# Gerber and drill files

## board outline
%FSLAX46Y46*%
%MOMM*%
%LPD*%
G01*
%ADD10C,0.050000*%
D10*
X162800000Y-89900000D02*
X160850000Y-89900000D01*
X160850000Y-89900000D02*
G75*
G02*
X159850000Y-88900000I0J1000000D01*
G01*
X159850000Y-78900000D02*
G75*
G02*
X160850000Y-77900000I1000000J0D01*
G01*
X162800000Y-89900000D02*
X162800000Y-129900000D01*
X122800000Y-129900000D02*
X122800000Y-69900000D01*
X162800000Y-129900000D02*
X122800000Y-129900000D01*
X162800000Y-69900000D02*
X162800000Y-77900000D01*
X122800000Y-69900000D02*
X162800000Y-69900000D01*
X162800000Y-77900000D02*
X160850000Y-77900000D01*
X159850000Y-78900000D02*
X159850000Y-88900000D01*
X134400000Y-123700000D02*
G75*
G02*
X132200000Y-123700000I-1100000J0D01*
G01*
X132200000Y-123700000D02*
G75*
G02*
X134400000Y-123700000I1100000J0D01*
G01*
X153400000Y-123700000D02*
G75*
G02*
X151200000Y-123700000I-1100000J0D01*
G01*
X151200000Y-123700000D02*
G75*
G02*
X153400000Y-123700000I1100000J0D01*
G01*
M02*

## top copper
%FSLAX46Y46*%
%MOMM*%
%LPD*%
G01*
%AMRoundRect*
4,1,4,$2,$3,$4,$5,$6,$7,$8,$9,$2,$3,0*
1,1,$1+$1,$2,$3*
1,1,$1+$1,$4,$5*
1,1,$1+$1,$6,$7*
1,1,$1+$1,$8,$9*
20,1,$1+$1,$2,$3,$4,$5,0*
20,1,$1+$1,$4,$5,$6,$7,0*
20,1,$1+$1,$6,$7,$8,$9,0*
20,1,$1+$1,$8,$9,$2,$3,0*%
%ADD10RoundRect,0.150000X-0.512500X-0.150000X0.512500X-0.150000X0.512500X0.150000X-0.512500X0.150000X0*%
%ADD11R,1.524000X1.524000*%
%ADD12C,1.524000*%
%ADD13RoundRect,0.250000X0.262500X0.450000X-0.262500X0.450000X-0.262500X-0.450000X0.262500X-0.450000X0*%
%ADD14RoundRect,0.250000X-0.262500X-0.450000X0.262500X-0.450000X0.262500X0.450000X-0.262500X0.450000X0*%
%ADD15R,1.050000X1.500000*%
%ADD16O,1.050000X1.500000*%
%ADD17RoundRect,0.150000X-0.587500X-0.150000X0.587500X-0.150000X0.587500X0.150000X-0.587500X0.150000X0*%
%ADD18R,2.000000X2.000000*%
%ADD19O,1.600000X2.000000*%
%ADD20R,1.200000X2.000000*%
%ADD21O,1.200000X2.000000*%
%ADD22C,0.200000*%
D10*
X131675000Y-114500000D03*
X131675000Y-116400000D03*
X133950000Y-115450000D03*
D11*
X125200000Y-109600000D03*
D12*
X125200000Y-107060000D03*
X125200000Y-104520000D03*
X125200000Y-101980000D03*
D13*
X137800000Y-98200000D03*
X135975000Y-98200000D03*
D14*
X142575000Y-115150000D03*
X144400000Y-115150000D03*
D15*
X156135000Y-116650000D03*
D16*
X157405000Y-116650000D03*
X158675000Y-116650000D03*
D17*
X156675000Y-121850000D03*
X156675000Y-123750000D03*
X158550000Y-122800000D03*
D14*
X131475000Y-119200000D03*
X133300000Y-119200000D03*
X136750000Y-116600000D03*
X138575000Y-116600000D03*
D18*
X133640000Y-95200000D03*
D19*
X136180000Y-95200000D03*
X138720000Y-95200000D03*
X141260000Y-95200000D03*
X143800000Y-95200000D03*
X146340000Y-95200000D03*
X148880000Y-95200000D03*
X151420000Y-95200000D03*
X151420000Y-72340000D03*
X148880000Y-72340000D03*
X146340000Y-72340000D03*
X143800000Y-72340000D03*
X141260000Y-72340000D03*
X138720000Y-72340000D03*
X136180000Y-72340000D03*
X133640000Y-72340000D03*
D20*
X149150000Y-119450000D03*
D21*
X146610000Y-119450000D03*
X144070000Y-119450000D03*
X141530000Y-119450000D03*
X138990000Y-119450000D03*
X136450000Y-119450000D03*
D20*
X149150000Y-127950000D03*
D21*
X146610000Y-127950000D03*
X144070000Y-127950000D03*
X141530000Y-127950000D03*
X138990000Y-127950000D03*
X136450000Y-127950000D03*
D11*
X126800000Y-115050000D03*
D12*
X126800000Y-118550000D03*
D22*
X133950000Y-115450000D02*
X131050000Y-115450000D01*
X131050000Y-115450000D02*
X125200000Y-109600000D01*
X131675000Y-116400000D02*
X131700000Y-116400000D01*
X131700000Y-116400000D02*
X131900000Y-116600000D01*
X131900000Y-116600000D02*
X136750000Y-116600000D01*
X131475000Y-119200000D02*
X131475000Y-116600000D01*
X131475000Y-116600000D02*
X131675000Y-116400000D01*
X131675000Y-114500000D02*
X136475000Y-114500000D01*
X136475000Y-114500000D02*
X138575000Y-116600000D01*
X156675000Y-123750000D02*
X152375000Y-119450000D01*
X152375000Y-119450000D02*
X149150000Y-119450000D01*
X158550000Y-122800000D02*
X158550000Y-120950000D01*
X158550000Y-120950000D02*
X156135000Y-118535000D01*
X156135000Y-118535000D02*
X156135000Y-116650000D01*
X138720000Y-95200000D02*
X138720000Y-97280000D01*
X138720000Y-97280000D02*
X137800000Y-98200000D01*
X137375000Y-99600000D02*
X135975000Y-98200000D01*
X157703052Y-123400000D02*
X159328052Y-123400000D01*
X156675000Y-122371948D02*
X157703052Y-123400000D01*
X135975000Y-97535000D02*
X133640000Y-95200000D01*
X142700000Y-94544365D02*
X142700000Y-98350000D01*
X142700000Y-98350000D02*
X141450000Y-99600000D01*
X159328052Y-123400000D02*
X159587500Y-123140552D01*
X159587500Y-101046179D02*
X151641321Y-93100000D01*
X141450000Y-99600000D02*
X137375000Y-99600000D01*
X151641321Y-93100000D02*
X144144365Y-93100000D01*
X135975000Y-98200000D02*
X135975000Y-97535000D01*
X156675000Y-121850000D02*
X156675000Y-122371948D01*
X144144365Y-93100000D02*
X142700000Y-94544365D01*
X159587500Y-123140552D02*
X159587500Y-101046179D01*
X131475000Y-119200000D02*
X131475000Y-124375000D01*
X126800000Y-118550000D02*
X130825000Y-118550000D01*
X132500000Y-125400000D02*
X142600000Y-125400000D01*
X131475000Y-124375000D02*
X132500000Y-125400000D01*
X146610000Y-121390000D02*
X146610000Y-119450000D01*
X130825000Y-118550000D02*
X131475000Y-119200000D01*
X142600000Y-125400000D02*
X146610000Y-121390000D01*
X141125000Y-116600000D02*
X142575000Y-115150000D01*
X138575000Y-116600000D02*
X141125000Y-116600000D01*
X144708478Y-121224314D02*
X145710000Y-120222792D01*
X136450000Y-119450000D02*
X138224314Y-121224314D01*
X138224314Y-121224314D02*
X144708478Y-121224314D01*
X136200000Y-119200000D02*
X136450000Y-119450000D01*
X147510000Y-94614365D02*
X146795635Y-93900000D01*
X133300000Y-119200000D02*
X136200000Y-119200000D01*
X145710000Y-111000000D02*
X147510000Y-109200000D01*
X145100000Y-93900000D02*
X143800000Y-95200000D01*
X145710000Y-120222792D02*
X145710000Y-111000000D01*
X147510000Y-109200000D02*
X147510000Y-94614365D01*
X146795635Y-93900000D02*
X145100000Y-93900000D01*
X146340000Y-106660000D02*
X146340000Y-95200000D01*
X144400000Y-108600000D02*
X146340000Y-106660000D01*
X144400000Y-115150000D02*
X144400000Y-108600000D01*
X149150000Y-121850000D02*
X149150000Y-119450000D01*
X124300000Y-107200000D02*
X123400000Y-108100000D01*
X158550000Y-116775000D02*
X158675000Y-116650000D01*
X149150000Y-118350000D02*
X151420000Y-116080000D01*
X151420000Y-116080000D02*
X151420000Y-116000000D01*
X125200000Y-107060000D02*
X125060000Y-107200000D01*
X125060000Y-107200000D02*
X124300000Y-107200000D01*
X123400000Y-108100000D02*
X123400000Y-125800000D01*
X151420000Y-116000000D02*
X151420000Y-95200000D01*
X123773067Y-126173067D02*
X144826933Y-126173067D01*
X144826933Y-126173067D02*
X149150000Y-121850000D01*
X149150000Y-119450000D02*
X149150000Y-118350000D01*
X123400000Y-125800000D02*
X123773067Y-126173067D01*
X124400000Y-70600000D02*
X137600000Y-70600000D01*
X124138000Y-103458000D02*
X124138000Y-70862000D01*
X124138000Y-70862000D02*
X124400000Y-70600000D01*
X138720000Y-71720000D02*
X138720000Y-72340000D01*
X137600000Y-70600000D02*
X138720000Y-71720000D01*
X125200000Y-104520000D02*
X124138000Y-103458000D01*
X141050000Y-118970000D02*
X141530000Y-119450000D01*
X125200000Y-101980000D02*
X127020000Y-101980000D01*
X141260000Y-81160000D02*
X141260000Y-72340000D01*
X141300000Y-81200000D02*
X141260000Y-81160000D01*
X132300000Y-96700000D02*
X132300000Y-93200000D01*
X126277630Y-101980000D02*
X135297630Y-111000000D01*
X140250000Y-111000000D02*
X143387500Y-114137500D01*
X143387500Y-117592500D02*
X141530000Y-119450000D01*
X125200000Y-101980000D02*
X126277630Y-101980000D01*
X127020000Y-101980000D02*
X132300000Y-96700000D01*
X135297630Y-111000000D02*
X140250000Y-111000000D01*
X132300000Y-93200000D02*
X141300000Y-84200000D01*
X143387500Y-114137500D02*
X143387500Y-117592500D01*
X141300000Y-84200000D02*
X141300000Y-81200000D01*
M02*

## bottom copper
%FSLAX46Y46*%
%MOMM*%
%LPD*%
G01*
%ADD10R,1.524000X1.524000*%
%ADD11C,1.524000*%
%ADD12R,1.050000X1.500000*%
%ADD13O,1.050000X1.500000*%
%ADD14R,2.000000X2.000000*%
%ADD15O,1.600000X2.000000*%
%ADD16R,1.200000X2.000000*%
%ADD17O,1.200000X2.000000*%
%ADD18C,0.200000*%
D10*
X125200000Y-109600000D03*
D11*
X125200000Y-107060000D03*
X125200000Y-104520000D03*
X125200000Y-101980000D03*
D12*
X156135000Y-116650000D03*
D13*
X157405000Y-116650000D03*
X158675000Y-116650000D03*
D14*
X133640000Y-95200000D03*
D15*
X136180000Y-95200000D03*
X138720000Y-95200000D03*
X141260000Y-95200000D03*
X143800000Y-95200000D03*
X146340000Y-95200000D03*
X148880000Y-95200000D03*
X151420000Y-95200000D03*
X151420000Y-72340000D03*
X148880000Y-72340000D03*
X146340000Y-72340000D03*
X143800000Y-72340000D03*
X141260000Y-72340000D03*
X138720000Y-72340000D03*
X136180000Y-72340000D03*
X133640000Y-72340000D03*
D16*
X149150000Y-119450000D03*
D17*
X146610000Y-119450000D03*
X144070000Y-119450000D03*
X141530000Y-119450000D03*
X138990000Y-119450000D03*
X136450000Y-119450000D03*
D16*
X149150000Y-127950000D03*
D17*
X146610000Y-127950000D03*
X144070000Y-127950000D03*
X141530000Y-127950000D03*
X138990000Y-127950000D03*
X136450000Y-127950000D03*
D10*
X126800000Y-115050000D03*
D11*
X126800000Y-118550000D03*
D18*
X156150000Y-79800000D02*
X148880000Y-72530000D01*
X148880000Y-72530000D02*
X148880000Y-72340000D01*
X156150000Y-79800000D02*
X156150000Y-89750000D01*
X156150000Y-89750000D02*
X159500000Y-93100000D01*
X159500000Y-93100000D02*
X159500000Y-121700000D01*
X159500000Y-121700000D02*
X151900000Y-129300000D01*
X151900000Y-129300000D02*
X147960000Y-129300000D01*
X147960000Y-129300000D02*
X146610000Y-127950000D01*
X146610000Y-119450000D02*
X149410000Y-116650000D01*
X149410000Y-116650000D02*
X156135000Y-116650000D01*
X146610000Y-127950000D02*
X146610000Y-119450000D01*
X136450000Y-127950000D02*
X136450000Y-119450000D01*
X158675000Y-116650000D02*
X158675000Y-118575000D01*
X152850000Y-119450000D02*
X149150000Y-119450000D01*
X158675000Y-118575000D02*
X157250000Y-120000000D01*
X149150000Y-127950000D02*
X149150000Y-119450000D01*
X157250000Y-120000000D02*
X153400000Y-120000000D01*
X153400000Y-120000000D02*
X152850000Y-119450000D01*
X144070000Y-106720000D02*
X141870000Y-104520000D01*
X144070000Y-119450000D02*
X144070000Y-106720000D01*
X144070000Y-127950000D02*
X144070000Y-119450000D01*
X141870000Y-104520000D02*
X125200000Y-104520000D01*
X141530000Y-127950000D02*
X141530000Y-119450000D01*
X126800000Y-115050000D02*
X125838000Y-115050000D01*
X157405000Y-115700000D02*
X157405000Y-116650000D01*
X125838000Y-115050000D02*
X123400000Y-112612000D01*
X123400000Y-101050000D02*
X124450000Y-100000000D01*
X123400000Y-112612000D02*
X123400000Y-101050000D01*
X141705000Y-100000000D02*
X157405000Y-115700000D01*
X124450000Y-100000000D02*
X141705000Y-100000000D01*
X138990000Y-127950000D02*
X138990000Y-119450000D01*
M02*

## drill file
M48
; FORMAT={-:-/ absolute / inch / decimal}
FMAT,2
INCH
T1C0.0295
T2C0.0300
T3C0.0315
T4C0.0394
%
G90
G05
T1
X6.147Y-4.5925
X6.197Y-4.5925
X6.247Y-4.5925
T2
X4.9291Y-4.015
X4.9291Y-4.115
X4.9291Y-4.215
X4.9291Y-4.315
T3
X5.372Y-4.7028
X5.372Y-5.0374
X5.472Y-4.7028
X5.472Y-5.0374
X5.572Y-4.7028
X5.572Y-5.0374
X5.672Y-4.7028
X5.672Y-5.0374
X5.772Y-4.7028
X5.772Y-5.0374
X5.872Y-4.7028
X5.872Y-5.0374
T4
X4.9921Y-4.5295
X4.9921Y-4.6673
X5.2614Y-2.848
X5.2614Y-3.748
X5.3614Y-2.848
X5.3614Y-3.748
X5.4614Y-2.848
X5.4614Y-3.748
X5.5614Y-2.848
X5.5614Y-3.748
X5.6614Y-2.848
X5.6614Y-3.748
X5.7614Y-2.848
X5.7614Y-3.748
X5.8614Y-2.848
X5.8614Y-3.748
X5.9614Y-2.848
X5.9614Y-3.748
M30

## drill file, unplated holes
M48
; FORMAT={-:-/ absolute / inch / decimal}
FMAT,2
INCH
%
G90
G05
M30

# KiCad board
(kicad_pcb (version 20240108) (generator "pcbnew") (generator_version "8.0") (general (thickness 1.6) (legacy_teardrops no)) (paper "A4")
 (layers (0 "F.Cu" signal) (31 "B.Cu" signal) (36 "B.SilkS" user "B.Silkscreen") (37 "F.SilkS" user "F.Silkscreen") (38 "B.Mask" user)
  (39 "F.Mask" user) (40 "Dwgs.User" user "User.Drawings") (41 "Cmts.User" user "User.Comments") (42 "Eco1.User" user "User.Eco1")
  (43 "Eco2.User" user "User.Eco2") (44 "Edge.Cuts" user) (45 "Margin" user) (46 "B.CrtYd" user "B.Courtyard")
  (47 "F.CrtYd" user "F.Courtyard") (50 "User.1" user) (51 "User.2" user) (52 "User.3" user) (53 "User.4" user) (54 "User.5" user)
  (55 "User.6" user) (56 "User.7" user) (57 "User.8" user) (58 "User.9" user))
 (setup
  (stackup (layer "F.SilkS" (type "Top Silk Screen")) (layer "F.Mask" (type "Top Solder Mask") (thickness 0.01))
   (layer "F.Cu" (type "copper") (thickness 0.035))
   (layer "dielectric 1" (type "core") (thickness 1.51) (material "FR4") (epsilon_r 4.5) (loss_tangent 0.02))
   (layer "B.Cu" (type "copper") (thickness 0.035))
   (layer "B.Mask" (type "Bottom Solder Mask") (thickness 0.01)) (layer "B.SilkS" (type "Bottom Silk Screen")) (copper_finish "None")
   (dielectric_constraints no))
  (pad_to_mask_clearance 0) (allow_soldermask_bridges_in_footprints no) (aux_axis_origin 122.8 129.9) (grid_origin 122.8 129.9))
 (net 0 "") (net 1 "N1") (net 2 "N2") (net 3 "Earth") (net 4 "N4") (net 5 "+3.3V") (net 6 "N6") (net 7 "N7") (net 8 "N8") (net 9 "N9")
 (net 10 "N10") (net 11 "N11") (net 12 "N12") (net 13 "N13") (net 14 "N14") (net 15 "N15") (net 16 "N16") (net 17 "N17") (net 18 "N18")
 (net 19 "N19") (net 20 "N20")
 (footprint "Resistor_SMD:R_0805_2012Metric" (layer "F.Cu") (at 143.4875 115.15)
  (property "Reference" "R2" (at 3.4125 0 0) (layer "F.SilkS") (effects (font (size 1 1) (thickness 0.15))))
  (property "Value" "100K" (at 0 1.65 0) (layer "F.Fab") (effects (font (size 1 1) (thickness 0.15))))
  (pad "1" smd roundrect (at -0.9125 0) (size 1.025 1.4) (layers "F.Cu" "F.Paste" "F.Mask") (roundrect_rratio 0.243902) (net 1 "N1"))
  (pad "2" smd roundrect (at 0.9125 0) (size 1.025 1.4) (layers "F.Cu" "F.Paste" "F.Mask") (roundrect_rratio 0.243902) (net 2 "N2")))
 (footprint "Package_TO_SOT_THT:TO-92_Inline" (layer "F.Cu") (at 156.135 116.65)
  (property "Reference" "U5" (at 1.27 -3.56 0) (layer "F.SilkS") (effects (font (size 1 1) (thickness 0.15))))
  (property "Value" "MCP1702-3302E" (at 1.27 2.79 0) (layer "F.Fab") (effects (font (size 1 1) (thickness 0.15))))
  (pad "1" thru_hole rect (at 0 0) (size 1.05 1.5) (drill 0.75) (layers "*.Cu" "*.Mask") (remove_unused_layers no) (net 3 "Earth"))
  (pad "2" thru_hole oval (at 1.27 0) (size 1.05 1.5) (drill 0.75) (layers "*.Cu" "*.Mask") (remove_unused_layers no) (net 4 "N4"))
  (pad "3" thru_hole oval (at 2.54 0) (size 1.05 1.5) (drill 0.75) (layers "*.Cu" "*.Mask") (remove_unused_layers no) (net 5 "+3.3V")))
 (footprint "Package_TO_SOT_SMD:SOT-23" (layer "F.Cu") (at 157.6125 122.8)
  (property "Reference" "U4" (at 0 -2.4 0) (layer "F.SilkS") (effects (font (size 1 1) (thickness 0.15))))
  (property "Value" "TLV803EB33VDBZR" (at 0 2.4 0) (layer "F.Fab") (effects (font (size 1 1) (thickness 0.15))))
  (pad "1" smd roundrect (at -0.9375 -0.95) (size 1.475 0.6) (layers "F.Cu" "F.Paste" "F.Mask") (roundrect_rratio 0.25) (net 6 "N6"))
  (pad "2" smd roundrect (at -0.9375 0.95) (size 1.475 0.6) (layers "F.Cu" "F.Paste" "F.Mask") (roundrect_rratio 0.25) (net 5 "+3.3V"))
  (pad "3" smd roundrect (at 0.9375 0) (size 1.475 0.6) (layers "F.Cu" "F.Paste" "F.Mask") (roundrect_rratio 0.25) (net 3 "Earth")))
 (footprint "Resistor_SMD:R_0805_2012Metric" (layer "F.Cu") (at 132.3875 119.2)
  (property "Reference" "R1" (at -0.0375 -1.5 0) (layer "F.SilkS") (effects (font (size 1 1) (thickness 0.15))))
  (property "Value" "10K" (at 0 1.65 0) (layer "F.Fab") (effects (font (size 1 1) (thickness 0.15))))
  (pad "1" smd roundrect (at -0.9125 0) (size 1.025 1.4) (layers "F.Cu" "F.Paste" "F.Mask") (roundrect_rratio 0.243902) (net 3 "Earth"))
  (pad "2" smd roundrect (at 0.9125 0) (size 1.025 1.4) (layers "F.Cu" "F.Paste" "F.Mask") (roundrect_rratio 0.243902) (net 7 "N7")))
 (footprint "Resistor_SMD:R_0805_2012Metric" (layer "F.Cu") (at 137.6625 116.6)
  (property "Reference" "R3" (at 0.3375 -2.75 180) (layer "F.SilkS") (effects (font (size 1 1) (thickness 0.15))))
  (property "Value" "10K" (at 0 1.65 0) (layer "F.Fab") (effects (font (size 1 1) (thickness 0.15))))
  (pad "1" smd roundrect (at -0.9125 0) (size 1.025 1.4) (layers "F.Cu" "F.Paste" "F.Mask") (roundrect_rratio 0.243902) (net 3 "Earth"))
  (pad "2" smd roundrect (at 0.9125 0) (size 1.025 1.4) (layers "F.Cu" "F.Paste" "F.Mask") (roundrect_rratio 0.243902) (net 1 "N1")))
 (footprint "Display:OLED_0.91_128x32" (layer "F.Cu") (at 125.1732 109.5902)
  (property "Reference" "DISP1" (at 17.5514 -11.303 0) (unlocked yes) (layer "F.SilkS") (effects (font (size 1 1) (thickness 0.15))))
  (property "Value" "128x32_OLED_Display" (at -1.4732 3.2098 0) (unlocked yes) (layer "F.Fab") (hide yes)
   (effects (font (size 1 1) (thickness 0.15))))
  (pad "1" thru_hole rect (at 0.0268 0.0098) (size 1.524 1.524) (drill 0.762) (layers "*.Cu" "*.Mask") (remove_unused_layers no)
   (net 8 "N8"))
  (pad "2" thru_hole circle (at 0.0268 -2.5302) (size 1.524 1.524) (drill 0.762) (layers "*.Cu" "*.Mask") (remove_unused_layers no)
   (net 5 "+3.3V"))
  (pad "3" thru_hole circle (at 0.0268 -5.0702) (size 1.524 1.524) (drill 0.762) (layers "*.Cu" "*.Mask") (remove_unused_layers no)
   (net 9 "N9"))
  (pad "4" thru_hole circle (at 0.0268 -7.6102) (size 1.524 1.524) (drill 0.762) (layers "*.Cu" "*.Mask") (remove_unused_layers no)
   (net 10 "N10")))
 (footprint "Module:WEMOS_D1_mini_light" (layer "F.Cu") (at 133.64 95.2 90)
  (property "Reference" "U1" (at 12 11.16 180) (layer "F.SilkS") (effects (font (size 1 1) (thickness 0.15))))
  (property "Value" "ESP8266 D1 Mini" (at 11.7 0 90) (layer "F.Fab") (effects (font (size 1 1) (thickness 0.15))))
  (pad "1" thru_hole rect (at 0 0 90) (size 2 2) (drill 1) (layers "*.Cu" "*.Mask") (remove_unused_layers no) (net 6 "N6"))
  (pad "2" thru_hole oval (at 0 2.54 90) (size 2 1.6) (drill 1) (layers "*.Cu" "*.Mask") (remove_unused_layers no) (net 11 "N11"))
  (pad "3" thru_hole oval (at 0 5.08 90) (size 2 1.6) (drill 1) (layers "*.Cu" "*.Mask") (remove_unused_layers no) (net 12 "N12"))
  (pad "4" thru_hole oval (at 0 7.62 90) (size 2 1.6) (drill 1) (layers "*.Cu" "*.Mask") (remove_unused_layers no) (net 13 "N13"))
  (pad "5" thru_hole oval (at 0 10.16 90) (size 2 1.6) (drill 1) (layers "*.Cu" "*.Mask") (remove_unused_layers no) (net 7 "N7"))
  (pad "6" thru_hole oval (at 0 12.7 90) (size 2 1.6) (drill 1) (layers "*.Cu" "*.Mask") (remove_unused_layers no) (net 2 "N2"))
  (pad "7" thru_hole oval (at 0 15.24 90) (size 2 1.6) (drill 1) (layers "*.Cu" "*.Mask") (remove_unused_layers no) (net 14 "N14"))
  (pad "8" thru_hole oval (at 0 17.78 90) (size 2 1.6) (drill 1) (layers "*.Cu" "*.Mask") (remove_unused_layers no) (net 5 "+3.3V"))
  (pad "9" thru_hole oval (at 22.86 17.78 90) (size 2 1.6) (drill 1) (layers "*.Cu" "*.Mask") (remove_unused_layers no) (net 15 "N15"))
  (pad "10" thru_hole oval (at 22.86 15.24 90) (size 2 1.6) (drill 1) (layers "*.Cu" "*.Mask") (remove_unused_layers no) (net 3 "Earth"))
  (pad "11" thru_hole oval (at 22.86 12.7 90) (size 2 1.6) (drill 1) (layers "*.Cu" "*.Mask") (remove_unused_layers no) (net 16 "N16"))
  (pad "12" thru_hole oval (at 22.86 10.16 90) (size 2 1.6) (drill 1) (layers "*.Cu" "*.Mask") (remove_unused_layers no) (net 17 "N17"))
  (pad "13" thru_hole oval (at 22.86 7.62 90) (size 2 1.6) (drill 1) (layers "*.Cu" "*.Mask") (remove_unused_layers no) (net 10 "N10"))
  (pad "14" thru_hole oval (at 22.86 5.08 90) (size 2 1.6) (drill 1) (layers "*.Cu" "*.Mask") (remove_unused_layers no) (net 9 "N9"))
  (pad "15" thru_hole oval (at 22.86 2.54 90) (size 2 1.6) (drill 1) (layers "*.Cu" "*.Mask") (remove_unused_layers no) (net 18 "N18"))
  (pad "16" thru_hole oval (at 22.86 0 90) (size 2 1.6) (drill 1) (layers "*.Cu" "*.Mask") (remove_unused_layers no) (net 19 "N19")))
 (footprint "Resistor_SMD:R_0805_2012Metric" (layer "F.Cu") (at 136.8875 98.2 180)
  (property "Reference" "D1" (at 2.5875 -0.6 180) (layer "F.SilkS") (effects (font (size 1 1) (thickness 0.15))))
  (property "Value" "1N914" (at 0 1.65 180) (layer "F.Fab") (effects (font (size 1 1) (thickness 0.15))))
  (pad "1" smd roundrect (at -0.9125 0 180) (size 1.025 1.4) (layers "F.Cu" "F.Paste" "F.Mask") (roundrect_rratio 0.243902) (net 12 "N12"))
  (pad "2" smd roundrect (at 0.9125 0 180) (size 1.025 1.4) (layers "F.Cu" "F.Paste" "F.Mask") (roundrect_rratio 0.243902) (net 6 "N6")))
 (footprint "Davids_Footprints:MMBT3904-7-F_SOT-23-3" (layer "F.Cu") (at 132.8125 115.45)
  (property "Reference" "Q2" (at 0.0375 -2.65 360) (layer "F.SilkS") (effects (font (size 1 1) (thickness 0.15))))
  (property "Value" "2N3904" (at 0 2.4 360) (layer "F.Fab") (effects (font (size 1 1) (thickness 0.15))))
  (pad "1" smd roundrect (at -1.1375 -0.95) (size 1.325 0.6) (layers "F.Cu" "F.Paste" "F.Mask") (roundrect_rratio 0.25) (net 1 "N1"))
  (pad "2" smd roundrect (at -1.1375 0.95) (size 1.325 0.6) (layers "F.Cu" "F.Paste" "F.Mask") (roundrect_rratio 0.25) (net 3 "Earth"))
  (pad "3" smd roundrect (at 1.1375 0) (size 1.325 0.6) (layers "F.Cu" "F.Paste" "F.Mask") (roundrect_rratio 0.25) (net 8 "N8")))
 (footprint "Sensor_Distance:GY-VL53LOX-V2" (layer "F.Cu") (at 142.8 119.45 180)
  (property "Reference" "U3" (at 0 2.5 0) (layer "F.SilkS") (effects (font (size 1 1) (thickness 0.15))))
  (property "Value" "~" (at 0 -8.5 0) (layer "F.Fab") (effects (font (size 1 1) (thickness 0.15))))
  (pad "1" thru_hole rect (at -6.35 0 180) (size 1.2 2) (drill 0.8) (layers "*.Cu" "*.Mask") (remove_unused_layers no) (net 5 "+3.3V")
   (thermal_bridge_angle 45))
  (pad "2" thru_hole oval (at -3.81 0 180) (size 1.2 2) (drill 0.8) (layers "*.Cu" "*.Mask") (remove_unused_layers no) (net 3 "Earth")
   (thermal_bridge_angle 45))
  (pad "3" thru_hole oval (at -1.27 0 180) (size 1.2 2) (drill 0.8) (layers "*.Cu" "*.Mask") (remove_unused_layers no) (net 9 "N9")
   (thermal_bridge_angle 45))
  (pad "4" thru_hole oval (at 1.27 0 180) (size 1.2 2) (drill 0.8) (layers "*.Cu" "*.Mask") (remove_unused_layers no) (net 10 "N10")
   (thermal_bridge_angle 45))
  (pad "5" thru_hole oval (at 3.81 0 180) (size 1.2 2) (drill 0.8) (layers "*.Cu" "*.Mask") (remove_unused_layers no) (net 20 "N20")
   (thermal_bridge_angle 45))
  (pad "6" thru_hole oval (at 6.35 0 180) (size 1.2 2) (drill 0.8) (layers "*.Cu" "*.Mask") (remove_unused_layers no) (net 7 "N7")
   (thermal_bridge_angle 45)))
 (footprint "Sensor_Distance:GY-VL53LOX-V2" (layer "B.Cu") (at 142.8 127.95 180)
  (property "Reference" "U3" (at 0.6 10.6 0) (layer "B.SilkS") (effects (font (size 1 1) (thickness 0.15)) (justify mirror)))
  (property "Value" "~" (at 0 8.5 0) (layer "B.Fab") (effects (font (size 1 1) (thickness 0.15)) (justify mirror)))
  (pad "1" thru_hole rect (at -6.35 0 180) (size 1.2 2) (drill 0.8) (layers "*.Cu" "*.Mask") (remove_unused_layers no) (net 5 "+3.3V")
   (thermal_bridge_angle 45))
  (pad "2" thru_hole oval (at -3.81 0 180) (size 1.2 2) (drill 0.8) (layers "*.Cu" "*.Mask") (remove_unused_layers no) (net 3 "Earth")
   (thermal_bridge_angle 45))
  (pad "3" thru_hole oval (at -1.27 0 180) (size 1.2 2) (drill 0.8) (layers "*.Cu" "*.Mask") (remove_unused_layers no) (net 9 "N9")
   (thermal_bridge_angle 45))
  (pad "4" thru_hole oval (at 1.27 0 180) (size 1.2 2) (drill 0.8) (layers "*.Cu" "*.Mask") (remove_unused_layers no) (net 10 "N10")
   (thermal_bridge_angle 45))
  (pad "5" thru_hole oval (at 3.81 0 180) (size 1.2 2) (drill 0.8) (layers "*.Cu" "*.Mask") (remove_unused_layers no) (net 20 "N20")
   (thermal_bridge_angle 45))
  (pad "6" thru_hole oval (at 6.35 0 180) (size 1.2 2) (drill 0.8) (layers "*.Cu" "*.Mask") (remove_unused_layers no) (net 7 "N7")
   (thermal_bridge_angle 45)))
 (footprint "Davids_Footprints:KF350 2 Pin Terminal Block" (layer "B.Cu") (at 126.8 115.05 -90)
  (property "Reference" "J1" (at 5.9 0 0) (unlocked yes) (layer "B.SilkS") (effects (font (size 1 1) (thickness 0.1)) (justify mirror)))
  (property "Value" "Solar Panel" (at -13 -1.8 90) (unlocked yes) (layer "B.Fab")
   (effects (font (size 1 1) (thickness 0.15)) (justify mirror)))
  (pad "1" thru_hole rect (at 0 0 270) (size 1.524 1.524) (drill 1) (layers "*.Cu" "*.Mask") (remove_unused_layers no) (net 4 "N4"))
  (pad "2" thru_hole circle (at 3.5 0 270) (size 1.524 1.524) (drill 1) (layers "*.Cu" "*.Mask") (remove_unused_layers no) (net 3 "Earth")))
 (gr_line (start 162.8 129.9) (end 122.8 129.9) (stroke (width 0.05) (type default)) (layer "Edge.Cuts"))
 (gr_line (start 162.8 69.9) (end 162.8 77.9) (stroke (width 0.05) (type default)) (layer "Edge.Cuts"))
 (gr_line (start 122.8 69.9) (end 162.8 69.9) (stroke (width 0.05) (type default)) (layer "Edge.Cuts"))
 (gr_arc (start 160.85 89.9) (mid 160.142893 89.607107) (end 159.85 88.9) (stroke (width 0.05) (type default)) (layer "Edge.Cuts"))
 (gr_line (start 159.85 78.9) (end 159.85 88.9) (stroke (width 0.05) (type default)) (layer "Edge.Cuts"))
 (gr_line (start 162.8 89.9) (end 162.8 129.9) (stroke (width 0.05) (type default)) (layer "Edge.Cuts"))
 (gr_line (start 122.8 129.9) (end 122.8 69.9) (stroke (width 0.05) (type default)) (layer "Edge.Cuts"))
 (gr_arc (start 159.85 78.9) (mid 160.142893 78.192893) (end 160.85 77.9) (stroke (width 0.05) (type default)) (layer "Edge.Cuts"))
 (gr_circle (center 133.3 123.7) (end 134.4 123.7) (stroke (width 0.05) (type default)) (fill none) (layer "Edge.Cuts"))
 (gr_line (start 162.8 89.9) (end 160.85 89.9) (stroke (width 0.05) (type default)) (layer "Edge.Cuts"))
 (gr_line (start 162.8 77.9) (end 160.85 77.9) (stroke (width 0.05) (type default)) (layer "Edge.Cuts"))
 (gr_circle (center 152.3 123.7) (end 153.4 123.7) (stroke (width 0.05) (type default)) (fill none) (layer "Edge.Cuts"))
 (segment (start 138.72 95.2) (end 138.72 97.28) (width 0.2) (layer "F.Cu") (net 12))
 (segment (start 138.72 97.28) (end 137.8 98.2) (width 0.2) (layer "F.Cu") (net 12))
 (segment (start 137.375 99.6) (end 135.975 98.2) (width 0.2) (layer "F.Cu") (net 6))
 (segment (start 157.703052 123.4) (end 159.328052 123.4) (width 0.2) (layer "F.Cu") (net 6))
 (segment (start 156.675 122.371948) (end 157.703052 123.4) (width 0.2) (layer "F.Cu") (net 6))
 (segment (start 135.975 97.535) (end 133.64 95.2) (width 0.2) (layer "F.Cu") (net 6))
 (segment (start 142.7 94.544365) (end 142.7 98.35) (width 0.2) (layer "F.Cu") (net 6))
 (segment (start 142.7 98.35) (end 141.45 99.6) (width 0.2) (layer "F.Cu") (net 6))
 (segment (start 159.328052 123.4) (end 159.5875 123.140552) (width 0.2) (layer "F.Cu") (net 6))
 (segment (start 159.5875 101.046179) (end 151.641321 93.1) (width 0.2) (layer "F.Cu") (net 6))
 (segment (start 141.45 99.6) (end 137.375 99.6) (width 0.2) (layer "F.Cu") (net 6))
 (segment (start 151.641321 93.1) (end 144.144365 93.1) (width 0.2) (layer "F.Cu") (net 6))
 (segment (start 135.975 98.2) (end 135.975 97.535) (width 0.2) (layer "F.Cu") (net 6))
 (segment (start 156.675 121.85) (end 156.675 122.371948) (width 0.2) (layer "F.Cu") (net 6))
 (segment (start 144.144365 93.1) (end 142.7 94.544365) (width 0.2) (layer "F.Cu") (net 6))
 (segment (start 159.5875 123.140552) (end 159.5875 101.046179) (width 0.2) (layer "F.Cu") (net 6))
 (segment (start 158.55 120.95) (end 156.135 118.535) (width 0.2) (layer "F.Cu") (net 3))
 (segment (start 158.55 122.8) (end 158.55 120.95) (width 0.2) (layer "F.Cu") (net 3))
 (segment (start 131.475 119.2) (end 131.475 124.375) (width 0.2) (layer "F.Cu") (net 3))
 (segment (start 126.8 118.55) (end 130.825 118.55) (width 0.2) (layer "F.Cu") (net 3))
 (segment (start 131.675 116.4) (end 131.7 116.4) (width 0.2) (layer "F.Cu") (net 3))
 (segment (start 156.135 118.535) (end 156.135 116.65) (width 0.2) (layer "F.Cu") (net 3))
 (segment (start 132.5 125.4) (end 142.6 125.4) (width 0.2) (layer "F.Cu") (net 3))
 (segment (start 131.475 124.375) (end 132.5 125.4) (width 0.2) (layer "F.Cu") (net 3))
 (segment (start 146.61 121.39) (end 146.61 119.45) (width 0.2) (layer "F.Cu") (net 3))
 (segment (start 130.825 118.55) (end 131.475 119.2) (width 0.2) (layer "F.Cu") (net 3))
 (segment (start 131.475 116.6) (end 131.675 116.4) (width 0.2) (layer "F.Cu") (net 3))
 (segment (start 131.475 119.2) (end 131.475 116.6) (width 0.2) (layer "F.Cu") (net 3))
 (segment (start 131.9 116.6) (end 136.75 116.6) (width 0.2) (layer "F.Cu") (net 3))
 (segment (start 142.6 125.4) (end 146.61 121.39) (width 0.2) (layer "F.Cu") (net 3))
 (segment (start 131.7 116.4) (end 131.9 116.6) (width 0.2) (layer "F.Cu") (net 3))
 (segment (start 147.96 129.3) (end 146.61 127.95) (width 0.2) (layer "B.Cu") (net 3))
 (segment (start 148.88 72.53) (end 148.88 72.34) (width 0.2) (layer "B.Cu") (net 3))
 (segment (start 159.5 121.7) (end 151.9 129.3) (width 0.2) (layer "B.Cu") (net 3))
 (segment (start 156.15 89.75) (end 159.5 93.1) (width 0.2) (layer "B.Cu") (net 3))
 (segment (start 149.41 116.65) (end 156.135 116.65) (width 0.2) (layer "B.Cu") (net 3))
 (segment (start 156.15 79.8) (end 156.15 89.75) (width 0.2) (layer "B.Cu") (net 3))
 (segment (start 156.15 79.8) (end 148.88 72.53) (width 0.2) (layer "B.Cu") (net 3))
 (segment (start 146.61 119.45) (end 149.41 116.65) (width 0.2) (layer "B.Cu") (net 3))
 (segment (start 159.5 93.1) (end 159.5 121.7) (width 0.2) (layer "B.Cu") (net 3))
 (segment (start 151.9 129.3) (end 147.96 129.3) (width 0.2) (layer "B.Cu") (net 3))
 (segment (start 146.61 127.95) (end 146.61 119.45) (width 0.2) (layer "B.Cu") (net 3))
 (segment (start 141.125 116.6) (end 142.575 115.15) (width 0.2) (layer "F.Cu") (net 1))
 (segment (start 138.575 116.6) (end 141.125 116.6) (width 0.2) (layer "F.Cu") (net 1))
 (segment (start 136.475 114.5) (end 138.575 116.6) (width 0.2) (layer "F.Cu") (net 1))
 (segment (start 131.675 114.5) (end 136.475 114.5) (width 0.2) (layer "F.Cu") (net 1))
 (segment (start 131.05 115.45) (end 125.2 109.6) (width 0.2) (layer "F.Cu") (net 8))
 (segment (start 133.95 115.45) (end 131.05 115.45) (width 0.2) (layer "F.Cu") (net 8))
 (segment (start 144.708478 121.224314) (end 145.71 120.222792) (width 0.2) (layer "F.Cu") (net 7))
 (segment (start 136.45 119.45) (end 138.224314 121.224314) (width 0.2) (layer "F.Cu") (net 7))
 (segment (start 138.224314 121.224314) (end 144.708478 121.224314) (width 0.2) (layer "F.Cu") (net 7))
 (segment (start 136.2 119.2) (end 136.45 119.45) (width 0.2) (layer "F.Cu") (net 7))
 (segment (start 147.51 94.614365) (end 146.795635 93.9) (width 0.2) (layer "F.Cu") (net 7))
 (segment (start 133.3 119.2) (end 136.2 119.2) (width 0.2) (layer "F.Cu") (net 7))
 (segment (start 145.71 111) (end 147.51 109.2) (width 0.2) (layer "F.Cu") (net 7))
 (segment (start 145.1 93.9) (end 143.8 95.2) (width 0.2) (layer "F.Cu") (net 7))
 (segment (start 145.71 120.222792) (end 145.71 111) (width 0.2) (layer "F.Cu") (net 7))
 (segment (start 147.51 109.2) (end 147.51 94.614365) (width 0.2) (layer "F.Cu") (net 7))
 (segment (start 146.795635 93.9) (end 145.1 93.9) (width 0.2) (layer "F.Cu") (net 7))
 (segment (start 136.45 127.95) (end 136.45 119.45) (width 0.2) (layer "B.Cu") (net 7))
 (segment (start 146.34 106.66) (end 146.34 95.2) (width 0.2) (layer "F.Cu") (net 2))
 (segment (start 144.4 108.6) (end 146.34 106.66) (width 0.2) (layer "F.Cu") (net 2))
 (segment (start 144.4 115.15) (end 144.4 108.6) (width 0.2) (layer "F.Cu") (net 2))
 (segment (start 149.15 121.85) (end 149.15 119.45) (width 0.2) (layer "F.Cu") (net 5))
 (segment (start 124.3 107.2) (end 123.4 108.1) (width 0.2) (layer "F.Cu") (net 5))
 (segment (start 152.375 119.45) (end 149.15 119.45) (width 0.2) (layer "F.Cu") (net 5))
 (segment (start 158.55 116.775) (end 158.675 116.65) (width 0.2) (layer "F.Cu") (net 5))
 (segment (start 149.15 118.35) (end 151.42 116.08) (width 0.2) (layer "F.Cu") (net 5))
 (segment (start 151.42 116.08) (end 151.42 116) (width 0.2) (layer "F.Cu") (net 5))
 (segment (start 125.2 107.06) (end 125.06 107.2) (width 0.2) (layer "F.Cu") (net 5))
 (segment (start 125.06 107.2) (end 124.3 107.2) (width 0.2) (layer "F.Cu") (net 5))
 (segment (start 156.675 123.75) (end 152.375 119.45) (width 0.2) (layer "F.Cu") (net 5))
 (segment (start 123.4 108.1) (end 123.4 125.8) (width 0.2) (layer "F.Cu") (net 5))
 (segment (start 151.42 116) (end 151.42 95.2) (width 0.2) (layer "F.Cu") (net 5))
 (segment (start 123.773067 126.173067) (end 144.826933 126.173067) (width 0.2) (layer "F.Cu") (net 5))
 (segment (start 144.826933 126.173067) (end 149.15 121.85) (width 0.2) (layer "F.Cu") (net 5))
 (segment (start 149.15 119.45) (end 149.15 118.35) (width 0.2) (layer "F.Cu") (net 5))
 (segment (start 123.4 125.8) (end 123.773067 126.173067) (width 0.2) (layer "F.Cu") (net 5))
 (segment (start 158.675 116.65) (end 158.675 118.575) (width 0.2) (layer "B.Cu") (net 5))
 (segment (start 152.85 119.45) (end 149.15 119.45) (width 0.2) (layer "B.Cu") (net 5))
 (segment (start 158.675 118.575) (end 157.25 120) (width 0.2) (layer "B.Cu") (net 5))
 (segment (start 149.15 127.95) (end 149.15 119.45) (width 0.2) (layer "B.Cu") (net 5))
 (segment (start 157.25 120) (end 153.4 120) (width 0.2) (layer "B.Cu") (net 5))
 (segment (start 153.4 120) (end 152.85 119.45) (width 0.2) (layer "B.Cu") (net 5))
 (segment (start 124.4 70.6) (end 137.6 70.6) (width 0.2) (layer "F.Cu") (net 9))
 (segment (start 124.138 103.458) (end 124.138 70.862) (width 0.2) (layer "F.Cu") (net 9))
 (segment (start 124.138 70.862) (end 124.4 70.6) (width 0.2) (layer "F.Cu") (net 9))
 (segment (start 138.72 71.72) (end 138.72 72.34) (width 0.2) (layer "F.Cu") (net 9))
 (segment (start 137.6 70.6) (end 138.72 71.72) (width 0.2) (layer "F.Cu") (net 9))
 (segment (start 125.2 104.52) (end 124.138 103.458) (width 0.2) (layer "F.Cu") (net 9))
 (segment (start 144.07 106.72) (end 141.87 104.52) (width 0.2) (layer "B.Cu") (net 9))
 (segment (start 144.07 119.45) (end 144.07 106.72) (width 0.2) (layer "B.Cu") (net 9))
 (segment (start 144.07 127.95) (end 144.07 119.45) (width 0.2) (layer "B.Cu") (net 9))
 (segment (start 141.87 104.52) (end 125.2 104.52) (width 0.2) (layer "B.Cu") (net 9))
 (segment (start 141.05 118.97) (end 141.53 119.45) (width 0.2) (layer "F.Cu") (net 10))
 (segment (start 125.2 101.98) (end 127.02 101.98) (width 0.2) (layer "F.Cu") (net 10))
 (segment (start 141.26 81.16) (end 141.26 72.34) (width 0.2) (layer "F.Cu") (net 10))
 (segment (start 141.3 81.2) (end 141.26 81.16) (width 0.2) (layer "F.Cu") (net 10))
 (segment (start 132.3 96.7) (end 132.3 93.2) (width 0.2) (layer "F.Cu") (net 10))
 (segment (start 126.27763 101.98) (end 135.29763 111) (width 0.2) (layer "F.Cu") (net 10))
 (segment (start 140.25 111) (end 143.3875 114.1375) (width 0.2) (layer "F.Cu") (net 10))
 (segment (start 143.3875 117.5925) (end 141.53 119.45) (width 0.2) (layer "F.Cu") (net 10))
 (segment (start 125.2 101.98) (end 126.27763 101.98) (width 0.2) (layer "F.Cu") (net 10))
 (segment (start 127.02 101.98) (end 132.3 96.7) (width 0.2) (layer "F.Cu") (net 10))
 (segment (start 135.29763 111) (end 140.25 111) (width 0.2) (layer "F.Cu") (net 10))
 (segment (start 132.3 93.2) (end 141.3 84.2) (width 0.2) (layer "F.Cu") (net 10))
 (segment (start 143.3875 114.1375) (end 143.3875 117.5925) (width 0.2) (layer "F.Cu") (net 10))
 (segment (start 141.3 84.2) (end 141.3 81.2) (width 0.2) (layer "F.Cu") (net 10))
 (segment (start 141.53 127.95) (end 141.53 119.45) (width 0.2) (layer "B.Cu") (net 10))
 (segment (start 126.8 115.05) (end 125.838 115.05) (width 0.2) (layer "B.Cu") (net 4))
 (segment (start 157.405 115.7) (end 157.405 116.65) (width 0.2) (layer "B.Cu") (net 4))
 (segment (start 125.838 115.05) (end 123.4 112.612) (width 0.2) (layer "B.Cu") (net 4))
 (segment (start 123.4 101.05) (end 124.45 100) (width 0.2) (layer "B.Cu") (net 4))
 (segment (start 123.4 112.612) (end 123.4 101.05) (width 0.2) (layer "B.Cu") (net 4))
 (segment (start 141.705 100) (end 157.405 115.7) (width 0.2) (layer "B.Cu") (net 4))
 (segment (start 124.45 100) (end 141.705 100) (width 0.2) (layer "B.Cu") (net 4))
 (segment (start 138.99 127.95) (end 138.99 119.45) (width 0.2) (layer "B.Cu") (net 20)))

